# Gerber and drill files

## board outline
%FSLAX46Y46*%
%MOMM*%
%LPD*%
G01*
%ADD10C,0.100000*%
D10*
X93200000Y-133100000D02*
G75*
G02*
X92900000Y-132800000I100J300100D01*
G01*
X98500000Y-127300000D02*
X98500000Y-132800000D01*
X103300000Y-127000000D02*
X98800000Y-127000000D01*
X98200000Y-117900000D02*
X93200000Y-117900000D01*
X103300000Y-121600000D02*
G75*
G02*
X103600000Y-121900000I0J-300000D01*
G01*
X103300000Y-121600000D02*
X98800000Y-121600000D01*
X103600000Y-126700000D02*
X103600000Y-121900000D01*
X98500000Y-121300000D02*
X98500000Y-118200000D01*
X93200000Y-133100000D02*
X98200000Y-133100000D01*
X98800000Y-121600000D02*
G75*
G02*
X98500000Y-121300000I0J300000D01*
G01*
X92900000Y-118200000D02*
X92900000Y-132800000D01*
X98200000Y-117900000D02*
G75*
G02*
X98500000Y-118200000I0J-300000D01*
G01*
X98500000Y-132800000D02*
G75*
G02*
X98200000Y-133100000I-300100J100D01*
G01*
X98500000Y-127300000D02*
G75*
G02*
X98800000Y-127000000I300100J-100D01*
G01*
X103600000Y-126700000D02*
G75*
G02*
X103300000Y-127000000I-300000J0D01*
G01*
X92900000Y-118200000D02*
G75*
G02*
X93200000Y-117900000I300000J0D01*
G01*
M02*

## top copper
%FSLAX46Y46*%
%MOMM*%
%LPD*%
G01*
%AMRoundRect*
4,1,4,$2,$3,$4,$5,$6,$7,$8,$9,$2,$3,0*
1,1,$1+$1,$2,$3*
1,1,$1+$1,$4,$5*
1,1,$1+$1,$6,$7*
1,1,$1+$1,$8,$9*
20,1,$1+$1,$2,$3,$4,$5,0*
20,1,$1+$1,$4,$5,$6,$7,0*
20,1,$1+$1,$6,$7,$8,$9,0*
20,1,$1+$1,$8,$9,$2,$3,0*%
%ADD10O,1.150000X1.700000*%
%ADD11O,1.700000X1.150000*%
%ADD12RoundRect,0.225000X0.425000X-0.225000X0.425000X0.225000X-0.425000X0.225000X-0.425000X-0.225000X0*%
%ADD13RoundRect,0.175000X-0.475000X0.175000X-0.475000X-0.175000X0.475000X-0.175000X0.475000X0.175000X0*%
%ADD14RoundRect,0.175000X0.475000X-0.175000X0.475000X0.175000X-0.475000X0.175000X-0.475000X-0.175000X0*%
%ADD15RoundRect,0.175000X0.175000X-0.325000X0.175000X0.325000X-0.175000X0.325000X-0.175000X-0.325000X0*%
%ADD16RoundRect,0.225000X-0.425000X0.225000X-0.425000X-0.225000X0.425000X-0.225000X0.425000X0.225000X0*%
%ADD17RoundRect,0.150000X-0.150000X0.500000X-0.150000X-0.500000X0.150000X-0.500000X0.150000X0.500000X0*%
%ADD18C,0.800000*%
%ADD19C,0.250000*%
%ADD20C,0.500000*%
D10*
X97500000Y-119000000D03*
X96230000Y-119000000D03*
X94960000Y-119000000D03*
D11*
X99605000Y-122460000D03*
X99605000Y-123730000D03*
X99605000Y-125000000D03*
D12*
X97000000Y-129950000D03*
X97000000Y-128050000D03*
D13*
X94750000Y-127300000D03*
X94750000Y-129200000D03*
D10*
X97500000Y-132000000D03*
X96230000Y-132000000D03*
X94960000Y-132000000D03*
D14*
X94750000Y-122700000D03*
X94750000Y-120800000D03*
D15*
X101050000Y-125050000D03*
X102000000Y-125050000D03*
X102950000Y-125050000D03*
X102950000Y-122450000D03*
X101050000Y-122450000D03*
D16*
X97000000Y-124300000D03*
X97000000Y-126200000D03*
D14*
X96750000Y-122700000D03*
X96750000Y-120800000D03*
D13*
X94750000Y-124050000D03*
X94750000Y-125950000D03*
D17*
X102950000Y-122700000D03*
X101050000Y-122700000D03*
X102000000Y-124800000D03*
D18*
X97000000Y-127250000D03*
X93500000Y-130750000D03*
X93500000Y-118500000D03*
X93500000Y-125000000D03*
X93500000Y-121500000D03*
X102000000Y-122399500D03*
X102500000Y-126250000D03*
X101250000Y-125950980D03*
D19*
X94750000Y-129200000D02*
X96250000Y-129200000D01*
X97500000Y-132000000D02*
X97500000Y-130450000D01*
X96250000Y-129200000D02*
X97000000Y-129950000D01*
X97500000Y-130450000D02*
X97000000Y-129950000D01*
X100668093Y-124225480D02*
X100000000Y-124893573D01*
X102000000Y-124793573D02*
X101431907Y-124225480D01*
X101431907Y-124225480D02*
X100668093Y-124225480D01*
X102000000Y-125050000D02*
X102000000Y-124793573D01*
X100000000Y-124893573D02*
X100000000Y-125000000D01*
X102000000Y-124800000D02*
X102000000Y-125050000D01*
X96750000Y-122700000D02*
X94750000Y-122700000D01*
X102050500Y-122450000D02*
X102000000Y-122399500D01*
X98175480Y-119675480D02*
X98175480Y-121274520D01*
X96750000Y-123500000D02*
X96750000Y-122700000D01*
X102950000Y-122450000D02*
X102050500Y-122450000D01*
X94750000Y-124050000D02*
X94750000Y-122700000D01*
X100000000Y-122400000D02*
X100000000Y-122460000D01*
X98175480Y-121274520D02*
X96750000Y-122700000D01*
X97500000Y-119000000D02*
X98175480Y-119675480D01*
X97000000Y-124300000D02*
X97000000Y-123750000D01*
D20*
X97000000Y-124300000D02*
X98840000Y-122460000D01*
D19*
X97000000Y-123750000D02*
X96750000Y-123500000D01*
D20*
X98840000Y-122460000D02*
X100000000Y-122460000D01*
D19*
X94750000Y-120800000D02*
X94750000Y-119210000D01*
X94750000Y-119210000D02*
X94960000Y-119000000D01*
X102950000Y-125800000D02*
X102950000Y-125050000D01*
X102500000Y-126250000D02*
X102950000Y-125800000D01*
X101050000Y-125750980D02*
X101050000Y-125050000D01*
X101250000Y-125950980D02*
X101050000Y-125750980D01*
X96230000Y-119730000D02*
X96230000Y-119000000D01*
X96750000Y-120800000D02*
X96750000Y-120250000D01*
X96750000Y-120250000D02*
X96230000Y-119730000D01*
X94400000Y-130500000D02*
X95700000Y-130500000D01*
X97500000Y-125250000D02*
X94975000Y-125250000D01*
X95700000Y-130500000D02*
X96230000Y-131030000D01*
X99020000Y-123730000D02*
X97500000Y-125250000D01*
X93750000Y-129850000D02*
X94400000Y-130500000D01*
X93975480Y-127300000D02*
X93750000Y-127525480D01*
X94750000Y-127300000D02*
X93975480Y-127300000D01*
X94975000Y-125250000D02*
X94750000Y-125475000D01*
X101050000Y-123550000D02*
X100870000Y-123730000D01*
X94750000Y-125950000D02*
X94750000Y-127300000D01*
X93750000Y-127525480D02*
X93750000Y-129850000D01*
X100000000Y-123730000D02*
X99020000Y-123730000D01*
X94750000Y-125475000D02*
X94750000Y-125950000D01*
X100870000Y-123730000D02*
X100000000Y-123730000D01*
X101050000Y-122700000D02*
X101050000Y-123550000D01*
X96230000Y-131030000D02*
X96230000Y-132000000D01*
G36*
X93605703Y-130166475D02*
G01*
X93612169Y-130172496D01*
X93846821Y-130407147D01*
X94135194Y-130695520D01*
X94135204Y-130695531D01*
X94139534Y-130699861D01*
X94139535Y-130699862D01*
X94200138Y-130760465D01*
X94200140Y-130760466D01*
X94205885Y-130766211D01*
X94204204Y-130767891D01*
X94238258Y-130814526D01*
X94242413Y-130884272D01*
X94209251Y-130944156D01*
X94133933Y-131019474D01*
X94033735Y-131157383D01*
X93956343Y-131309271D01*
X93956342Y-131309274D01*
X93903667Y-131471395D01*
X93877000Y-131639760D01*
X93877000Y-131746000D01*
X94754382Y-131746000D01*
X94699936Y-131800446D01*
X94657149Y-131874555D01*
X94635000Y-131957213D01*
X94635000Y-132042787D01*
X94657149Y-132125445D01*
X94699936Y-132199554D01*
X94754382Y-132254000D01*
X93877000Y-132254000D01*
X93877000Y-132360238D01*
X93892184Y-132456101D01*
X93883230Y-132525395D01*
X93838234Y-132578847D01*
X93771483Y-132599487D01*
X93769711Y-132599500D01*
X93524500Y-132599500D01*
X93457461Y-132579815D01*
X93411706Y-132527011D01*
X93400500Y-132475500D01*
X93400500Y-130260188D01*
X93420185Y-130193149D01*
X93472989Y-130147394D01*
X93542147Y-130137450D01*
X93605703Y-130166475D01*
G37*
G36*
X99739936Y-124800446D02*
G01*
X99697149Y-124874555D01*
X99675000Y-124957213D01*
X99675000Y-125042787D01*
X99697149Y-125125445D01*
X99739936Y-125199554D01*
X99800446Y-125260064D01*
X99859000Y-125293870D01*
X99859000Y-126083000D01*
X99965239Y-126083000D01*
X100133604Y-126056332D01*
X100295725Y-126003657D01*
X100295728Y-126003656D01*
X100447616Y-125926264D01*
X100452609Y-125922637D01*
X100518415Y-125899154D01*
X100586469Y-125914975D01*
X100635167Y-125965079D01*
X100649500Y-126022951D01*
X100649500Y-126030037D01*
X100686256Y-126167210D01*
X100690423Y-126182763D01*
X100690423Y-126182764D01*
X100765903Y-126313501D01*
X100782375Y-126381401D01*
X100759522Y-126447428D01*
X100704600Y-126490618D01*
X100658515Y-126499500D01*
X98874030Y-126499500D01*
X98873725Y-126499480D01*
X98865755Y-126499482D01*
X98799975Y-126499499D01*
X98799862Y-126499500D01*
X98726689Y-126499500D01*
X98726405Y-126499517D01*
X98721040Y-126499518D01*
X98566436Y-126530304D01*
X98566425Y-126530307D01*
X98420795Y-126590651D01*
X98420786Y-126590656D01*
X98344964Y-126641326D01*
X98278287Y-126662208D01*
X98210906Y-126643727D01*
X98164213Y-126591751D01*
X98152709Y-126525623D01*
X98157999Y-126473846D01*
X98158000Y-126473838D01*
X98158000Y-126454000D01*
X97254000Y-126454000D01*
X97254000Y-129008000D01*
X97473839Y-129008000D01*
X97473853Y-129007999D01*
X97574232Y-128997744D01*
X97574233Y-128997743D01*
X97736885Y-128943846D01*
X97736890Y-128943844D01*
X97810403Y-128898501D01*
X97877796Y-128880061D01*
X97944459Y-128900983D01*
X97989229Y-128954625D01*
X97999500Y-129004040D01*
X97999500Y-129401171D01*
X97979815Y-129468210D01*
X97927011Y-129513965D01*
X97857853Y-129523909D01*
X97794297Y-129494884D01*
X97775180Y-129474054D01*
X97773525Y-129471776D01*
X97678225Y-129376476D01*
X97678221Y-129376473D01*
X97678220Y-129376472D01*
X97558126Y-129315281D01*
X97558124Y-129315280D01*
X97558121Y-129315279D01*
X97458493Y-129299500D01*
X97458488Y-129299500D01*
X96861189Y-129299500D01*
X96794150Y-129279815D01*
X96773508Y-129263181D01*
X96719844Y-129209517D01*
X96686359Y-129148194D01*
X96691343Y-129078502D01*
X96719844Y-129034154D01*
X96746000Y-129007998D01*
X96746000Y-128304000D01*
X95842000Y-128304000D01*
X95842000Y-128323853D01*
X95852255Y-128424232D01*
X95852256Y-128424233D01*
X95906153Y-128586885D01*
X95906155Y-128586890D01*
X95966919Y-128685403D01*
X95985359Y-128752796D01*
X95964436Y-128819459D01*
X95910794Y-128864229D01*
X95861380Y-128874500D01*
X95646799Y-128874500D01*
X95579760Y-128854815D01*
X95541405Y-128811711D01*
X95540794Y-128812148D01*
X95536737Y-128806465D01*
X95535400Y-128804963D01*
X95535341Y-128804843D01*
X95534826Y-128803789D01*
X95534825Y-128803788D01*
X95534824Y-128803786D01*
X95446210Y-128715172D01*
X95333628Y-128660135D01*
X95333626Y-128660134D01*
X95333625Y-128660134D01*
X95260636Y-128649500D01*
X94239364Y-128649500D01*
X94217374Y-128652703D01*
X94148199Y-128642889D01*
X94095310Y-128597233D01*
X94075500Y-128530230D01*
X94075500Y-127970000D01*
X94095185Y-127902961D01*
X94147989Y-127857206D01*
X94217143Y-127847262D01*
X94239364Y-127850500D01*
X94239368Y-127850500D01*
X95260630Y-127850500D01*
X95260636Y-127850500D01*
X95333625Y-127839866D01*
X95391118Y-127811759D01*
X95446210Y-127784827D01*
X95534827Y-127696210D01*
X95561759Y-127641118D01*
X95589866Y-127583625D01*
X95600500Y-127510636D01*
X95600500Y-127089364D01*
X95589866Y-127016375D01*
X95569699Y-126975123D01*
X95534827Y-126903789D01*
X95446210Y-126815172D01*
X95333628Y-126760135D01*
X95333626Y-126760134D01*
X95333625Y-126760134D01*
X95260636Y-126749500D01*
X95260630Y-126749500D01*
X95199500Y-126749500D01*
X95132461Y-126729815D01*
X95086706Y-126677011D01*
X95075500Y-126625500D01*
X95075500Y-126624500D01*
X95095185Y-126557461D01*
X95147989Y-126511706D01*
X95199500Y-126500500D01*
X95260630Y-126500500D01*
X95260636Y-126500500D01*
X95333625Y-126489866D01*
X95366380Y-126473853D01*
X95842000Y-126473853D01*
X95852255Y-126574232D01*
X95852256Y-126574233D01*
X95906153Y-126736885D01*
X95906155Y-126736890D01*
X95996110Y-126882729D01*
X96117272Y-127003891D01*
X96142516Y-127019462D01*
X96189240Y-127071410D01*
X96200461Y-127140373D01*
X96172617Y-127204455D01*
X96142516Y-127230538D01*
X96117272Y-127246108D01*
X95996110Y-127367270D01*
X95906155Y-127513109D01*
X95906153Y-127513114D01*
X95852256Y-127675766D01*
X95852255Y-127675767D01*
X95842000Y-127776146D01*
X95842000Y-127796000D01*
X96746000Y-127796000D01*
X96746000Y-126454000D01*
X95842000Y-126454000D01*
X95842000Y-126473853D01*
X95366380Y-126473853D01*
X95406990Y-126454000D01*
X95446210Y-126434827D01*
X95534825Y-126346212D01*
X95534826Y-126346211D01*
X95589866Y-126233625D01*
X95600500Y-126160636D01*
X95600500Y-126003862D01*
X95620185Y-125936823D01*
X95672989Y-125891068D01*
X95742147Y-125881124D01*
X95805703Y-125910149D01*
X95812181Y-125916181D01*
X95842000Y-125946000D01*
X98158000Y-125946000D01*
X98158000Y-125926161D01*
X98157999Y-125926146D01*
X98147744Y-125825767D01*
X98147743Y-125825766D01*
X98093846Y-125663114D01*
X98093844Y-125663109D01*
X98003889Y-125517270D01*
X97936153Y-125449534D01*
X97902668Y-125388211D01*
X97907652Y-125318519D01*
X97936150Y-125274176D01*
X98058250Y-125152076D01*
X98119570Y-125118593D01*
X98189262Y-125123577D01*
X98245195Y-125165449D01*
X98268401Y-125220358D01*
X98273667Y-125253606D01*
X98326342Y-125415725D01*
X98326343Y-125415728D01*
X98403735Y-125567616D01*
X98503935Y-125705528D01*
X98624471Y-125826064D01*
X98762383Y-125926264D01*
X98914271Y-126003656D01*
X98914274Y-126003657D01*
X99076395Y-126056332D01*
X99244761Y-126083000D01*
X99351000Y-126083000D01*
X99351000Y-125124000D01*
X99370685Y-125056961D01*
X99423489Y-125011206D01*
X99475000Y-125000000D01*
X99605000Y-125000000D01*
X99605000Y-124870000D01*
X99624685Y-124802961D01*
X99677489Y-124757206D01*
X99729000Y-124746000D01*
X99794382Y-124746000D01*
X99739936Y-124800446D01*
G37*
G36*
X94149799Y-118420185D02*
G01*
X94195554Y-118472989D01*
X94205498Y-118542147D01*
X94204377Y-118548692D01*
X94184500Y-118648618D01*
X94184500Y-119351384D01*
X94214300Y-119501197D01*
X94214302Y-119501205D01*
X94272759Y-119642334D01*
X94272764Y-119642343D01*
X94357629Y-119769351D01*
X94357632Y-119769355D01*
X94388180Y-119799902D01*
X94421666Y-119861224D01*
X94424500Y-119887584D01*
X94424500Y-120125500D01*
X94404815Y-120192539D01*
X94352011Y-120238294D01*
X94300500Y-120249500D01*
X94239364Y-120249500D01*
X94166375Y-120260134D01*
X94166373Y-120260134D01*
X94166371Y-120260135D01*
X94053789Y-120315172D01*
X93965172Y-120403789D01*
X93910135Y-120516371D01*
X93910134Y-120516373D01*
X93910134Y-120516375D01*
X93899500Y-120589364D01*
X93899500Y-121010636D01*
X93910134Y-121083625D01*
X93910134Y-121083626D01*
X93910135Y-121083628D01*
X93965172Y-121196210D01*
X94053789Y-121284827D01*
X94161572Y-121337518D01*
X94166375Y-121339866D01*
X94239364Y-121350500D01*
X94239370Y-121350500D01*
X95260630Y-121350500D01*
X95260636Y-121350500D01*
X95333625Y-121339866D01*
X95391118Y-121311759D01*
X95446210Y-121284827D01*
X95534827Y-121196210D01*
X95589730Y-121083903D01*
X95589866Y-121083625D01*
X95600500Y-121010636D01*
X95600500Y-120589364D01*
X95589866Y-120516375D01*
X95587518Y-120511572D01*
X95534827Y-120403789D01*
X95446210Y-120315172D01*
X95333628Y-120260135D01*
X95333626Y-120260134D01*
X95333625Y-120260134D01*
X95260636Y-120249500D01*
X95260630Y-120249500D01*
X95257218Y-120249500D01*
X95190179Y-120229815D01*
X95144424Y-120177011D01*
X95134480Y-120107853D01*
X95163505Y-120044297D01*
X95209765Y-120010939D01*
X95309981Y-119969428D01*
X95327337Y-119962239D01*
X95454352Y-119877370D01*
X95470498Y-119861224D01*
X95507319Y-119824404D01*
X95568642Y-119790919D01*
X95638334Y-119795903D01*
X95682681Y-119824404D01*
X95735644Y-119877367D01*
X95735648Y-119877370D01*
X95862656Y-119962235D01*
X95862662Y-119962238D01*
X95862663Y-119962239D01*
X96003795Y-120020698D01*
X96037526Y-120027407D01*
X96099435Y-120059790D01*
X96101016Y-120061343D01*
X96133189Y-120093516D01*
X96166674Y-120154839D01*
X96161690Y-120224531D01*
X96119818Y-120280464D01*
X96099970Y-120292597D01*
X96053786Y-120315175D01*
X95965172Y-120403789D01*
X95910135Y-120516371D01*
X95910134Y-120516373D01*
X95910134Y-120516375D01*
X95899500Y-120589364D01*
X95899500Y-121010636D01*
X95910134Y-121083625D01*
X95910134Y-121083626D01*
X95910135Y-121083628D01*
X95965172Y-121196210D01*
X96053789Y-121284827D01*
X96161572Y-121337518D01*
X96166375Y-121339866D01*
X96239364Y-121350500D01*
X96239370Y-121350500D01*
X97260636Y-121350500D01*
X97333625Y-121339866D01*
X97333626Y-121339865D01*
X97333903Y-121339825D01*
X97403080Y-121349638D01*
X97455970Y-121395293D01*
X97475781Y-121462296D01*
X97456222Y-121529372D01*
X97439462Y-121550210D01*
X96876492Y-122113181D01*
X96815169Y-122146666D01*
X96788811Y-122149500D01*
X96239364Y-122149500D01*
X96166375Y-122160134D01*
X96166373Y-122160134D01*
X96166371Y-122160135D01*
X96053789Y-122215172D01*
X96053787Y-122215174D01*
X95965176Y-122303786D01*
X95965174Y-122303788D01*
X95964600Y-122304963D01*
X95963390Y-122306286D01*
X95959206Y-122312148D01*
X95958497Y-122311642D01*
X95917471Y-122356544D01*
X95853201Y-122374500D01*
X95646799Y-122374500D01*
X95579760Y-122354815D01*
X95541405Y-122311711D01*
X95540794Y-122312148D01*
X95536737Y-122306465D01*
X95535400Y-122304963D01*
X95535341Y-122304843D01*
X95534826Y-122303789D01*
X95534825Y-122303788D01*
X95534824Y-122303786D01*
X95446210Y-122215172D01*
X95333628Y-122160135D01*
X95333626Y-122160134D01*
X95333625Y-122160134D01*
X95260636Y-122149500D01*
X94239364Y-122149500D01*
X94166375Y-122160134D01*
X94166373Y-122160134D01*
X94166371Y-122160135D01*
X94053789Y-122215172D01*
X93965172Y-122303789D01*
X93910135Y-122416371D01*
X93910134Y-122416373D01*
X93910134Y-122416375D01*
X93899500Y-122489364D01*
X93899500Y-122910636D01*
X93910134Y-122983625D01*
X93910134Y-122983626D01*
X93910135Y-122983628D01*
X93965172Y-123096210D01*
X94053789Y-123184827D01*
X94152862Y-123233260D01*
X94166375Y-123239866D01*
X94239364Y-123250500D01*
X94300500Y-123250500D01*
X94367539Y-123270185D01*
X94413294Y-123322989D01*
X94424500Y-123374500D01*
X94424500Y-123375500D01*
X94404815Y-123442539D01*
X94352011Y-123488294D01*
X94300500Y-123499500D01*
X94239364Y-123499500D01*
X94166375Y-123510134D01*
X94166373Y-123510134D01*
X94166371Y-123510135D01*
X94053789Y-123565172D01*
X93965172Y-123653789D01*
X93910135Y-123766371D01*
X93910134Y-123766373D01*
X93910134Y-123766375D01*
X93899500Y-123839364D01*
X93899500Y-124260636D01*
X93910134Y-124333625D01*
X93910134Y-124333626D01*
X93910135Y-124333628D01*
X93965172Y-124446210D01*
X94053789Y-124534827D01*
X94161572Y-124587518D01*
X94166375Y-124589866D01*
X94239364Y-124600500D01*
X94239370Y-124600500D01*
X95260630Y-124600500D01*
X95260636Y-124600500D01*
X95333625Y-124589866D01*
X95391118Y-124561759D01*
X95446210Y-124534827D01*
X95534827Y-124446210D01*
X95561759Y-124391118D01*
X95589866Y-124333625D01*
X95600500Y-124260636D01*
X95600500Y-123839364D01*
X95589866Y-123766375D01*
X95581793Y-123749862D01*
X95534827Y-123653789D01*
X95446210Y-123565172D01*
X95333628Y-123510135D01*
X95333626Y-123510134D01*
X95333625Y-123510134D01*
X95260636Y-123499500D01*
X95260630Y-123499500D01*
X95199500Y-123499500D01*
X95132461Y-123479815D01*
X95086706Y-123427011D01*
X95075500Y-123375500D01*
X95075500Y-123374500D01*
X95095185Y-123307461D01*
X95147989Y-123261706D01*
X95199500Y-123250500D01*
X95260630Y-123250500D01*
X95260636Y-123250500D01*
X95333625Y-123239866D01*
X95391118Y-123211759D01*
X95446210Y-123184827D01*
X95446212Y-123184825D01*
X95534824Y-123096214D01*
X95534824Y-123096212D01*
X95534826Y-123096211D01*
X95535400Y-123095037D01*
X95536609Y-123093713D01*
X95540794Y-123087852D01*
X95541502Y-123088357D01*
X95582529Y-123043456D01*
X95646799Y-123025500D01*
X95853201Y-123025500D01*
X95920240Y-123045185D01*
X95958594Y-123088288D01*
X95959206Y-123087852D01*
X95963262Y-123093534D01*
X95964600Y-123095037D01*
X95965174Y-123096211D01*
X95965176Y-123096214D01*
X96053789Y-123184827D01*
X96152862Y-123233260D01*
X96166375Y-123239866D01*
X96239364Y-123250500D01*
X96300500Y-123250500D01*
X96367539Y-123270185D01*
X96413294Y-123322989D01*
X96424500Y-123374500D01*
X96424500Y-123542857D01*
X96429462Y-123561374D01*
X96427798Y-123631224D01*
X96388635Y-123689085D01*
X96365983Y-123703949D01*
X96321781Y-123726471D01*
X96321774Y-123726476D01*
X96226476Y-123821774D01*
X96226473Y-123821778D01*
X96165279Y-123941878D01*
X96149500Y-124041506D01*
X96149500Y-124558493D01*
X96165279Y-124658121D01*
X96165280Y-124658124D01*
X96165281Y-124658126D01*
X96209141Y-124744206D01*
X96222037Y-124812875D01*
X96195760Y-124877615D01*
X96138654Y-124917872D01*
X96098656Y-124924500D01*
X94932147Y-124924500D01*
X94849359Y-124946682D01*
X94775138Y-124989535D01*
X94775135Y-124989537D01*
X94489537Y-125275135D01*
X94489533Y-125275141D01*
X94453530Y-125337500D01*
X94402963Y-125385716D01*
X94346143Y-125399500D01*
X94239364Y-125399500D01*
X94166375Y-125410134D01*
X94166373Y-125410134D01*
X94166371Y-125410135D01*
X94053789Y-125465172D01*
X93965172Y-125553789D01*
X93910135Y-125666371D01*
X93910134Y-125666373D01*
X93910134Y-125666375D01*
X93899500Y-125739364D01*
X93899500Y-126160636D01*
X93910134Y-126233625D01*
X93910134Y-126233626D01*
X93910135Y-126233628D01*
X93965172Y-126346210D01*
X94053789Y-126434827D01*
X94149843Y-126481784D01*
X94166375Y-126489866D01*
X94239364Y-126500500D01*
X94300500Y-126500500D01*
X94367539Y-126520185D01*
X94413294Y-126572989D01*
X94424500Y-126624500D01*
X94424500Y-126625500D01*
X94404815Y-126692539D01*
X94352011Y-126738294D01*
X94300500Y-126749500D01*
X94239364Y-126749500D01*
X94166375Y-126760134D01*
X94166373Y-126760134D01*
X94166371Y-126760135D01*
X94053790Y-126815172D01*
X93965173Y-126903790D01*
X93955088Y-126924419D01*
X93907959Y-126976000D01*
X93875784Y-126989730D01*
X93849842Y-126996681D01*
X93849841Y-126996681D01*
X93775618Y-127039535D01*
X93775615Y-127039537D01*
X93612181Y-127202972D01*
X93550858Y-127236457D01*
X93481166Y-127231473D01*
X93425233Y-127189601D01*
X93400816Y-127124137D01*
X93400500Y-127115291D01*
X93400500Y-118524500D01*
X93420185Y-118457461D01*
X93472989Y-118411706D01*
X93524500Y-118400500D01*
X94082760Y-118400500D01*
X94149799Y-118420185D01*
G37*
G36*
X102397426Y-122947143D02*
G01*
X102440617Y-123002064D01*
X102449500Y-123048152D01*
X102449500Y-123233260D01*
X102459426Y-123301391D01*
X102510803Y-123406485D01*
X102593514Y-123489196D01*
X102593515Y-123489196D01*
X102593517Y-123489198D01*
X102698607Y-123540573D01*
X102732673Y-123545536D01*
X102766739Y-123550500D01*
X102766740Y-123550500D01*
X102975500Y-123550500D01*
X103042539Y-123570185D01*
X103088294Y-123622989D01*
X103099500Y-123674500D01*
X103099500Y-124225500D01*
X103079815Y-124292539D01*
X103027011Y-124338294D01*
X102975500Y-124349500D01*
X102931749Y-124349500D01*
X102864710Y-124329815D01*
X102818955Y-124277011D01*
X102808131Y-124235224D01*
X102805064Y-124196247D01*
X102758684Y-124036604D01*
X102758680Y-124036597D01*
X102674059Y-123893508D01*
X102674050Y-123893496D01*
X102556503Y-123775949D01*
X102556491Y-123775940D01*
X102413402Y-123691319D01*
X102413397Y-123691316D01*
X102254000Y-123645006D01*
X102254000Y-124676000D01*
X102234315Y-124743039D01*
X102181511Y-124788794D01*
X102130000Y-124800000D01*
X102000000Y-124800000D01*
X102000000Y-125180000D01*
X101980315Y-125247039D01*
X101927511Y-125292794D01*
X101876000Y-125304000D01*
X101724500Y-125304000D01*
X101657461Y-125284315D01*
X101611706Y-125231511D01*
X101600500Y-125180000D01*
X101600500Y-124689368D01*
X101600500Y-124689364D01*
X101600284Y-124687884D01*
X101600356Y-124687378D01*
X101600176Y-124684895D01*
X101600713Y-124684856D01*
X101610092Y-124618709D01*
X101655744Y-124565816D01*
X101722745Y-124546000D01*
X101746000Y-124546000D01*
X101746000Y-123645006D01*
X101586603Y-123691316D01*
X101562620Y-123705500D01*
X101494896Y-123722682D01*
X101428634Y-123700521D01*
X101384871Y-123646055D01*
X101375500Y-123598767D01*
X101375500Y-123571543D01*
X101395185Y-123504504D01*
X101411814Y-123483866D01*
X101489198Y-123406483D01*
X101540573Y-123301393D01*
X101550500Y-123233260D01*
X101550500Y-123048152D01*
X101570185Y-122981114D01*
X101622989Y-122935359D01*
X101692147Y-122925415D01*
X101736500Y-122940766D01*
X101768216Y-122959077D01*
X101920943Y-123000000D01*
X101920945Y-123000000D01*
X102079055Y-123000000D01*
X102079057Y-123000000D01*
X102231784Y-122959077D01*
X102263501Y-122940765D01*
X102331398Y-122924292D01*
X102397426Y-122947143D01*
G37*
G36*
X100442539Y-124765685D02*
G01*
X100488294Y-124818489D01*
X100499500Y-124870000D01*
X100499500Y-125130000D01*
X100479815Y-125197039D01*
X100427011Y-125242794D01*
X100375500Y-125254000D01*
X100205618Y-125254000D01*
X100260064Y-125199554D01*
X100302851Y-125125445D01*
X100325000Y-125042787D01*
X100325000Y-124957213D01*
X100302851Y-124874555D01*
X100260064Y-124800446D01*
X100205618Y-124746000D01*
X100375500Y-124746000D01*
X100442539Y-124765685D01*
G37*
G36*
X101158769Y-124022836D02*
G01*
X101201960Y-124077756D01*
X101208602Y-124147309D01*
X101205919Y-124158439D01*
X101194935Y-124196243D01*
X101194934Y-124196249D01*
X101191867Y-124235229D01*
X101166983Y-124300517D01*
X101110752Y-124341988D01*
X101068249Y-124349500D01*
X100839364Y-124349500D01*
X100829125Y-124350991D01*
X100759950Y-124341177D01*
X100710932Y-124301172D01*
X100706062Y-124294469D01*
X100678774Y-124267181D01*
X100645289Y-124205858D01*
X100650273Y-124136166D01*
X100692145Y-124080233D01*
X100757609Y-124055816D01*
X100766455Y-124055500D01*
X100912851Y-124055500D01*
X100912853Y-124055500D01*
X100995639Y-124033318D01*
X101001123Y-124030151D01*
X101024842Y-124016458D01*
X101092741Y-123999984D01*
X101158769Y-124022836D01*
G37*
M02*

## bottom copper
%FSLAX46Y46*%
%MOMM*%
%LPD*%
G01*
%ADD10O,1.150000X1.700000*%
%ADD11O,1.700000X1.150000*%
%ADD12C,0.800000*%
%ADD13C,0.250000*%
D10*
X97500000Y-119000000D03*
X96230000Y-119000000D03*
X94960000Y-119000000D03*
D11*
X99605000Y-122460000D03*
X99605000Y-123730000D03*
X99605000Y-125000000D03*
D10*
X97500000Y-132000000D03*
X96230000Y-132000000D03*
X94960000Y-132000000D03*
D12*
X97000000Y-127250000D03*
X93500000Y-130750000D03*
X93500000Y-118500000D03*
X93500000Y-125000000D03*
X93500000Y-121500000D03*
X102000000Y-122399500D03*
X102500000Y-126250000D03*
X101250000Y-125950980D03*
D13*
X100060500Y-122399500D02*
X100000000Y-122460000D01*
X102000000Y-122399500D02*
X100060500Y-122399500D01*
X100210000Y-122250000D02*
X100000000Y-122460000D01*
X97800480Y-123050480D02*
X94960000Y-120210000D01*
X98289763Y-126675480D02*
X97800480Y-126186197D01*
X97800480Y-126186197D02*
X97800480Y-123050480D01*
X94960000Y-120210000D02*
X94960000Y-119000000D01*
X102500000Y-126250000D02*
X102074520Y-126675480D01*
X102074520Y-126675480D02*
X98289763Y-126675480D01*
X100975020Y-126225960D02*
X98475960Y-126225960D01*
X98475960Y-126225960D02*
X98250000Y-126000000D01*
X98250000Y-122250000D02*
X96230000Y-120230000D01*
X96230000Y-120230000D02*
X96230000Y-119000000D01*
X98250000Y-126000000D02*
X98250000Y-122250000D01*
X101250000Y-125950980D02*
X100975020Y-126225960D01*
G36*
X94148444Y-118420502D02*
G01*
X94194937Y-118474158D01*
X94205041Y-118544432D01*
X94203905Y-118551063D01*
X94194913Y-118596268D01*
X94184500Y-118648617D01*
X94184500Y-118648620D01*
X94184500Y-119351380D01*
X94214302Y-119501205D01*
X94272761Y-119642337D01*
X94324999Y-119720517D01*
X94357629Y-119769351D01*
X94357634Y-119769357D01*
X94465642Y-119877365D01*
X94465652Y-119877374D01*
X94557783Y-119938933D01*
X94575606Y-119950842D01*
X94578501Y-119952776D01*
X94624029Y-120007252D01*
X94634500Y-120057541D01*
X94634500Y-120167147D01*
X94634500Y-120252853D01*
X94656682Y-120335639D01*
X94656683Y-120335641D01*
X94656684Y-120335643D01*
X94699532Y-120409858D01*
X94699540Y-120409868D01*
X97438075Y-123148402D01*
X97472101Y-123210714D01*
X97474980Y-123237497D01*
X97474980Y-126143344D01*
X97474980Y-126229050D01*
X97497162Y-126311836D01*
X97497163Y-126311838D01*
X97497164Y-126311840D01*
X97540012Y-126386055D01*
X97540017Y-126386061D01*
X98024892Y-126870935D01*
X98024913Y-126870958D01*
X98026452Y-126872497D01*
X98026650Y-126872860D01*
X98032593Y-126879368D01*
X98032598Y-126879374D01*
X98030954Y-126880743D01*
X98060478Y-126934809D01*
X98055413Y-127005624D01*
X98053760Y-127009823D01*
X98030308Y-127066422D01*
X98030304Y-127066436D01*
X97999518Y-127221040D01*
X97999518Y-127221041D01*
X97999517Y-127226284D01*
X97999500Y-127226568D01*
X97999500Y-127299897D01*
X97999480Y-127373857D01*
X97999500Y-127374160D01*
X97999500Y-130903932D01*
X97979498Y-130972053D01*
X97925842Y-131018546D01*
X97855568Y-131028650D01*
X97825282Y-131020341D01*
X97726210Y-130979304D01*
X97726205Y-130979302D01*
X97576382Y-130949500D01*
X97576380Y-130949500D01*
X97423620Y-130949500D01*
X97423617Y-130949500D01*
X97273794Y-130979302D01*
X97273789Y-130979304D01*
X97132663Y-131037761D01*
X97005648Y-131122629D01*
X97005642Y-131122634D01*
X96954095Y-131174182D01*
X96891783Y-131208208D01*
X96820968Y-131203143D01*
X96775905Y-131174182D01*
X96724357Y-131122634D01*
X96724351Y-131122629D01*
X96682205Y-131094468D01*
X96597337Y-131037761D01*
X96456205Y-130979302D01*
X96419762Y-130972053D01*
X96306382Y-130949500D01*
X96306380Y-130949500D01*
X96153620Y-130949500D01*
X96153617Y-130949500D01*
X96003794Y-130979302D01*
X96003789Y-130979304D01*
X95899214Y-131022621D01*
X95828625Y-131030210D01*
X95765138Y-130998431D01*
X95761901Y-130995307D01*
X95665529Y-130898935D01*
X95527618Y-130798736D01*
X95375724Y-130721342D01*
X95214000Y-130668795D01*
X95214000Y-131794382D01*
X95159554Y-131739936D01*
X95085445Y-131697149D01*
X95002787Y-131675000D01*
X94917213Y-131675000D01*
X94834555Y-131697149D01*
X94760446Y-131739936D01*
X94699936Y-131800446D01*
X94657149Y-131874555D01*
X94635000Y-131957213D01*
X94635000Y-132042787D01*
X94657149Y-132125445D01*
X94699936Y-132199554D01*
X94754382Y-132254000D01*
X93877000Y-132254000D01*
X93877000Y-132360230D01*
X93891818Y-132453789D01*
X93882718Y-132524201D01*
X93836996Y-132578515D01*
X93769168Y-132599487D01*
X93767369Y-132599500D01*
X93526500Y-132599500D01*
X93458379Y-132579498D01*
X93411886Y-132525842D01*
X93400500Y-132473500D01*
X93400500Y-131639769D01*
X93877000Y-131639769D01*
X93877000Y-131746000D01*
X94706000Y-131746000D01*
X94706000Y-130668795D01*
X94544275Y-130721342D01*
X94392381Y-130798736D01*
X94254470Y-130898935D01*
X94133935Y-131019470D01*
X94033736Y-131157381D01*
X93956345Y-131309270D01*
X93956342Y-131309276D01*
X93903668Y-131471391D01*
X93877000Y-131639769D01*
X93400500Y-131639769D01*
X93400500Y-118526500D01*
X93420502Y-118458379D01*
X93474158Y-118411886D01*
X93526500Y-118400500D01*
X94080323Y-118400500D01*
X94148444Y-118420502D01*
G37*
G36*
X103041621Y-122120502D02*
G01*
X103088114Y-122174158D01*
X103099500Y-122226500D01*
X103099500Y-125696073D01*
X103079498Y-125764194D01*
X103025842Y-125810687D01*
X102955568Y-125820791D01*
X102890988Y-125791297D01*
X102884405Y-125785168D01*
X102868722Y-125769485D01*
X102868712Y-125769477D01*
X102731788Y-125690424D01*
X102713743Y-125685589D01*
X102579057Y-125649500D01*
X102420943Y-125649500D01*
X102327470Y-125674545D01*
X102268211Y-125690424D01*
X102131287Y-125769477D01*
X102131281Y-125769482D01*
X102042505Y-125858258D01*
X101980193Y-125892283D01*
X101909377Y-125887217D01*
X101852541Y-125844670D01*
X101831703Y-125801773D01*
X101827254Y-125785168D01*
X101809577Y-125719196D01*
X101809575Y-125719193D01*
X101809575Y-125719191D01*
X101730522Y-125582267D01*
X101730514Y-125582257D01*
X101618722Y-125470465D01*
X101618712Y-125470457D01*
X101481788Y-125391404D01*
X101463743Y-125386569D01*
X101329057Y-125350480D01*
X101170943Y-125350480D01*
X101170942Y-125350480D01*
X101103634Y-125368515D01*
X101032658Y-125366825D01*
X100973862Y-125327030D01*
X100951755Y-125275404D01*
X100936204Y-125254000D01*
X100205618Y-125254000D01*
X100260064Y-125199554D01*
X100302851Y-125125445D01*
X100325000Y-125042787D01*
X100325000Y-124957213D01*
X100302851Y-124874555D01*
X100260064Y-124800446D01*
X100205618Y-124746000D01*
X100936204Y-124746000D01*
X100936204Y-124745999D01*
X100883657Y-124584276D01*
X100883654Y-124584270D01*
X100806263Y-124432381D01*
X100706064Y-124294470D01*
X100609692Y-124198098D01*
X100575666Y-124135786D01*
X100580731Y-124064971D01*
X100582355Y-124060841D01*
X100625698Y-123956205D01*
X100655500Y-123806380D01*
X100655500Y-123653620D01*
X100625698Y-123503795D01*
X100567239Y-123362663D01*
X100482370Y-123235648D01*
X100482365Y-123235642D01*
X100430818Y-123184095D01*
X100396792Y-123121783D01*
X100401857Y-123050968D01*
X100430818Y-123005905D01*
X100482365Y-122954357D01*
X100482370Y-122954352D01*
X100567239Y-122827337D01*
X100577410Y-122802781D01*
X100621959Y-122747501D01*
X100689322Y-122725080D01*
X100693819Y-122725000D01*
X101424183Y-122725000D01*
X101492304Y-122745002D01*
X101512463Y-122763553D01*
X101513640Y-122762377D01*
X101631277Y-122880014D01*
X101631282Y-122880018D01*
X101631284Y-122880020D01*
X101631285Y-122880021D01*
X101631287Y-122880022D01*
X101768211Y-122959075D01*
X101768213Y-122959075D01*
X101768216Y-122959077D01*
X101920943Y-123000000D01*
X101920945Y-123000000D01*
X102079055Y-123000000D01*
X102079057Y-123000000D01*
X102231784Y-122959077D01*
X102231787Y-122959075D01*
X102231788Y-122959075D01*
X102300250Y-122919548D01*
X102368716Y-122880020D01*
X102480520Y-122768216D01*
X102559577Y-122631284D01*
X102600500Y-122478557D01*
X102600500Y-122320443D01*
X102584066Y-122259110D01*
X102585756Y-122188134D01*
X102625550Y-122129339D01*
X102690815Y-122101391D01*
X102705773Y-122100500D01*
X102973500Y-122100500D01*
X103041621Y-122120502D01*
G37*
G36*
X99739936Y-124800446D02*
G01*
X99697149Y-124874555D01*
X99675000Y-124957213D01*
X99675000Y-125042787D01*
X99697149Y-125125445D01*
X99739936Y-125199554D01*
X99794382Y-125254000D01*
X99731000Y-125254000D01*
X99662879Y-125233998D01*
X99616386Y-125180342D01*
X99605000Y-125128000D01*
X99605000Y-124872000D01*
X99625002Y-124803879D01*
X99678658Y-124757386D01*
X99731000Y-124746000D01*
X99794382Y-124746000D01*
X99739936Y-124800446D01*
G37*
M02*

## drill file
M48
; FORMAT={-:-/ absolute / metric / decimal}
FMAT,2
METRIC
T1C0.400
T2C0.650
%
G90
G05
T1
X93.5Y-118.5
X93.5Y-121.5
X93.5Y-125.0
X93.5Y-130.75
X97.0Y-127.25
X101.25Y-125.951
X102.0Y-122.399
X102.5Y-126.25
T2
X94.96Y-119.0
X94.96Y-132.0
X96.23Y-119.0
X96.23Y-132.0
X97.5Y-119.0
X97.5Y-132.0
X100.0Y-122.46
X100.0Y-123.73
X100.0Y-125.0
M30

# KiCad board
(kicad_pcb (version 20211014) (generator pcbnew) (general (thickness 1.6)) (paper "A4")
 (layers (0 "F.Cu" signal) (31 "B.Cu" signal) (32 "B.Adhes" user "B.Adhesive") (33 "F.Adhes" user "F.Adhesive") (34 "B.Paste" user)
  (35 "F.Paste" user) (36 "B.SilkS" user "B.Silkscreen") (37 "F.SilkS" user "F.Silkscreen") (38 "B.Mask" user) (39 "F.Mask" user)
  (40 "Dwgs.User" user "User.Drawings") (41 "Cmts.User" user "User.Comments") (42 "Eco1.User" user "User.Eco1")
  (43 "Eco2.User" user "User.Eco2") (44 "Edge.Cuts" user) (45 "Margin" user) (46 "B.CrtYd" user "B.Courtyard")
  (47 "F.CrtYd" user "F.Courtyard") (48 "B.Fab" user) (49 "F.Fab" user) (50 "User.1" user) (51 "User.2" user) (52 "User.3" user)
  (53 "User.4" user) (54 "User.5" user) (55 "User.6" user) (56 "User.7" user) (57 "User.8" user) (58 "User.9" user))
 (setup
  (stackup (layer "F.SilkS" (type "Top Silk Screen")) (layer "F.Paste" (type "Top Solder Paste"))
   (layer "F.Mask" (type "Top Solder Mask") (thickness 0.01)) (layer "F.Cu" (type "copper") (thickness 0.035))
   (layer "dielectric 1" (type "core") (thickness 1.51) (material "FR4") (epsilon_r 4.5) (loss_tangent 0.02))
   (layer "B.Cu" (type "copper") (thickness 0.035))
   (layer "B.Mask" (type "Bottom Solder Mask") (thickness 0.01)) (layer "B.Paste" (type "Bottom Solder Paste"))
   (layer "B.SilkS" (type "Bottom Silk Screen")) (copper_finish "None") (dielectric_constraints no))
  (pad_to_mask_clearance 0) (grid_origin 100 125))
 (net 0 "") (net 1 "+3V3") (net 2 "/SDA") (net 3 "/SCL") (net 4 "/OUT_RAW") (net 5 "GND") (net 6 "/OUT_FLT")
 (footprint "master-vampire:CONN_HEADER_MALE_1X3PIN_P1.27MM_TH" (layer "F.Cu") (at 97.5 119 180)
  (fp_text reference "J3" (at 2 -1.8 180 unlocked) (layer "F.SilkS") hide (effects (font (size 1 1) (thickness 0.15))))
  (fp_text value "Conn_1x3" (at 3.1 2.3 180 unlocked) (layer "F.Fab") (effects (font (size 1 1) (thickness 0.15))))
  (pad "1" thru_hole oval (at 0 0 180) (size 1.15 1.7) (drill 0.65) (layers *.Cu *.Mask) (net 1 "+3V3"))
  (pad "2" thru_hole oval (at 1.27 0 180) (size 1.15 1.7) (drill 0.65) (layers *.Cu *.Mask) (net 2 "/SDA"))
  (pad "3" thru_hole oval (at 2.54 0 180) (size 1.15 1.7) (drill 0.65) (layers *.Cu *.Mask) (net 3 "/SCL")))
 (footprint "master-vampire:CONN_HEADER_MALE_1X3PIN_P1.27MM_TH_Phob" (layer "F.Cu") (at 100 122.46 -90)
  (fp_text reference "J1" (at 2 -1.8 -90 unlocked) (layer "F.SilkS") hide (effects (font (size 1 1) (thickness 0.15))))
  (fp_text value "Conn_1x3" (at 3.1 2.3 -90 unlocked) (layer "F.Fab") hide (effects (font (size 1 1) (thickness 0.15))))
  (pad "1" thru_hole oval (at 0 0 270) (size 1.15 1.7) (drill 0.65 (offset 0 0.395)) (layers *.Cu *.Mask) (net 1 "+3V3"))
  (pad "2" thru_hole oval (at 1.27 0 270) (size 1.15 1.7) (drill 0.65 (offset 0 0.395)) (layers *.Cu *.Mask) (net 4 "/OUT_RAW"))
  (pad "3" thru_hole oval (at 2.54 0 270) (size 1.15 1.7) (drill 0.65 (offset 0 0.395)) (layers *.Cu *.Mask) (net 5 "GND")))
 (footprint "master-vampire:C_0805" (layer "F.Cu") (at 97 129 90)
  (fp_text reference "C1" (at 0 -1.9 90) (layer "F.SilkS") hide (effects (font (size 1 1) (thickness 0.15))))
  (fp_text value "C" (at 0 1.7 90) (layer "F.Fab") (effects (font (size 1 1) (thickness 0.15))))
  (pad "1" smd roundrect (at -0.95 0 90) (size 0.9 1.3) (layers "F.Cu" "F.Paste" "F.Mask") (roundrect_rratio 0.25) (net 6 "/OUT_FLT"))
  (pad "2" smd roundrect (at 0.95 0 90) (size 0.9 1.3) (layers "F.Cu" "F.Paste" "F.Mask") (roundrect_rratio 0.25) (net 5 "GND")))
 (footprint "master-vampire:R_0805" (layer "F.Cu") (at 94.75 128.25 -90)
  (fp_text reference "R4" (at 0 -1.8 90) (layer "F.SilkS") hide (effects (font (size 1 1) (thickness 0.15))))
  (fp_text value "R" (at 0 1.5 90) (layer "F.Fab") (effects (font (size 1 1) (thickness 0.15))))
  (pad "1" smd roundrect (at -0.95 0 270) (size 0.7 1.3) (layers "F.Cu" "F.Paste" "F.Mask") (roundrect_rratio 0.25) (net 4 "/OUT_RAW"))
  (pad "2" smd roundrect (at 0.95 0 270) (size 0.7 1.3) (layers "F.Cu" "F.Paste" "F.Mask") (roundrect_rratio 0.25) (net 6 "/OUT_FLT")))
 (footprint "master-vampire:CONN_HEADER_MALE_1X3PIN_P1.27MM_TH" (layer "F.Cu") (at 97.5 132 180)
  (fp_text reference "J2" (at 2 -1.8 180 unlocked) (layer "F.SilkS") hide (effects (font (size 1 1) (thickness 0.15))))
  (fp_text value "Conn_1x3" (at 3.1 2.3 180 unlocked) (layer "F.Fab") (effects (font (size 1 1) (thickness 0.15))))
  (pad "1" thru_hole oval (at 0 0 180) (size 1.15 1.7) (drill 0.65) (layers *.Cu *.Mask) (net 6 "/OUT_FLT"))
  (pad "2" thru_hole oval (at 1.27 0 180) (size 1.15 1.7) (drill 0.65) (layers *.Cu *.Mask) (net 4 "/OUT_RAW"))
  (pad "3" thru_hole oval (at 2.54 0 180) (size 1.15 1.7) (drill 0.65) (layers *.Cu *.Mask) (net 5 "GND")))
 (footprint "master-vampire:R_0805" (layer "F.Cu") (at 94.75 121.75 90)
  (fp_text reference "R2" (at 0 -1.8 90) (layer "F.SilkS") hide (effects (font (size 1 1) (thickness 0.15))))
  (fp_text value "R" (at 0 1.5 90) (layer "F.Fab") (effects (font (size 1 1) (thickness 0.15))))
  (pad "1" smd roundrect (at -0.95 0 90) (size 0.7 1.3) (layers "F.Cu" "F.Paste" "F.Mask") (roundrect_rratio 0.25) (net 1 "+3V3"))
  (pad "2" smd roundrect (at 0.95 0 90) (size 0.7 1.3) (layers "F.Cu" "F.Paste" "F.Mask") (roundrect_rratio 0.25) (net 3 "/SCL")))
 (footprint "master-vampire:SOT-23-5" (layer "F.Cu") (at 102 123.75 90)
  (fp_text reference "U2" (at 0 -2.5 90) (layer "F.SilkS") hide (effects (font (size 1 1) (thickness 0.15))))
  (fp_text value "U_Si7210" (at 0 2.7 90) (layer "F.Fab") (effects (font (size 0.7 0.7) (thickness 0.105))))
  (pad "1" smd roundrect (at -1.3 -0.95 90) (size 1 0.7) (layers "F.Cu" "F.Paste" "F.Mask") (roundrect_rratio 0.25) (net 2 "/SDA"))
  (pad "2" smd roundrect (at -1.3 0 90) (size 1 0.7) (layers "F.Cu" "F.Paste" "F.Mask") (roundrect_rratio 0.25) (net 5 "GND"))
  (pad "3" smd roundrect (at -1.3 0.95 90) (size 1 0.7) (layers "F.Cu" "F.Paste" "F.Mask") (roundrect_rratio 0.25) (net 3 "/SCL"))
  (pad "4" smd roundrect (at 1.3 0.95 90) (size 1 0.7) (layers "F.Cu" "F.Paste" "F.Mask") (roundrect_rratio 0.25) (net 1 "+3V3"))
  (pad "5" smd roundrect (at 1.3 -0.95 90) (size 1 0.7) (layers "F.Cu" "F.Paste" "F.Mask") (roundrect_rratio 0.25) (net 4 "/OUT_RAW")))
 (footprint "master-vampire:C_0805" (layer "F.Cu") (at 97 125.25 -90)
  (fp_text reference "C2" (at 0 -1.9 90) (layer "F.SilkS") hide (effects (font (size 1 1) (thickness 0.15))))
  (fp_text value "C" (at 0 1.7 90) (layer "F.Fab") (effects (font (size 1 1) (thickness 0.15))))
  (pad "1" smd roundrect (at -0.95 0 270) (size 0.9 1.3) (layers "F.Cu" "F.Paste" "F.Mask") (roundrect_rratio 0.25) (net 1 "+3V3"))
  (pad "2" smd roundrect (at 0.95 0 270) (size 0.9 1.3) (layers "F.Cu" "F.Paste" "F.Mask") (roundrect_rratio 0.25) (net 5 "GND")))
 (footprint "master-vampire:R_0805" (layer "F.Cu") (at 96.75 121.75 90)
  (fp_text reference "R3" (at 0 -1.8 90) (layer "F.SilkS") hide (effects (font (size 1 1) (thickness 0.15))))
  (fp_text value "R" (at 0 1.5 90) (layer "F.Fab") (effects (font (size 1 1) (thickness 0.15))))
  (pad "1" smd roundrect (at -0.95 0 90) (size 0.7 1.3) (layers "F.Cu" "F.Paste" "F.Mask") (roundrect_rratio 0.25) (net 1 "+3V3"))
  (pad "2" smd roundrect (at 0.95 0 90) (size 0.7 1.3) (layers "F.Cu" "F.Paste" "F.Mask") (roundrect_rratio 0.25) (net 2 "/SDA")))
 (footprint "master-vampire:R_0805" (layer "F.Cu") (at 94.75 125 -90)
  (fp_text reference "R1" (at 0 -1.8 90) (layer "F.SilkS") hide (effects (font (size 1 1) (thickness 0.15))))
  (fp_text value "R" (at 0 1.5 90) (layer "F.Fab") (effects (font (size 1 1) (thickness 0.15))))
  (pad "1" smd roundrect (at -0.95 0 270) (size 0.7 1.3) (layers "F.Cu" "F.Paste" "F.Mask") (roundrect_rratio 0.25) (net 1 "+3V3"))
  (pad "2" smd roundrect (at 0.95 0 270) (size 0.7 1.3) (layers "F.Cu" "F.Paste" "F.Mask") (roundrect_rratio 0.25) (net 4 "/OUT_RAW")))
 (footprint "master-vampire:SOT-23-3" (layer "F.Cu") (at 102 123.75 -90)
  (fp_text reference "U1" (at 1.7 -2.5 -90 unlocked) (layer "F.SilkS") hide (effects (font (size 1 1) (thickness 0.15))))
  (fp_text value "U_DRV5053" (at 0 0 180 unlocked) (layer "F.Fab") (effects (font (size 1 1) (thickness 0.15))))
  (pad "1" smd roundrect (at -1.05 -0.95 270) (size 1.3 0.6) (layers "F.Cu" "F.Paste" "F.Mask") (roundrect_rratio 0.25) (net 1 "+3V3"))
  (pad "2" smd roundrect (at -1.05 0.95 270) (size 1.3 0.6) (layers "F.Cu" "F.Paste" "F.Mask") (roundrect_rratio 0.25) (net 4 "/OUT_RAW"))
  (pad "3" smd roundrect (at 1.05 0 270) (size 1.3 0.6) (layers "F.Cu" "F.Paste" "F.Mask") (roundrect_rratio 0.25) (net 5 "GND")))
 (gr_arc (start 93.2 133.1) (mid 92.987897 133.012103) (end 92.9 132.8) (layer "Edge.Cuts") (width 0.1))
 (gr_line (start 98.5 127.3) (end 98.5 132.8) (layer "Edge.Cuts") (width 0.1))
 (gr_line (start 103.3 127) (end 98.8 127) (layer "Edge.Cuts") (width 0.1))
 (gr_line (start 98.2 117.9) (end 93.2 117.9) (layer "Edge.Cuts") (width 0.1))
 (gr_arc (start 103.3 121.6) (mid 103.512132 121.687868) (end 103.6 121.9) (layer "Edge.Cuts") (width 0.1))
 (gr_line (start 103.3 121.6) (end 98.8 121.6) (layer "Edge.Cuts") (width 0.1))
 (gr_line (start 103.6 126.7) (end 103.6 121.9) (layer "Edge.Cuts") (width 0.1))
 (gr_line (start 98.5 121.3) (end 98.5 118.2) (layer "Edge.Cuts") (width 0.1))
 (gr_line (start 93.2 133.1) (end 98.2 133.1) (layer "Edge.Cuts") (width 0.1))
 (gr_arc (start 98.8 121.6) (mid 98.587868 121.512132) (end 98.5 121.3) (layer "Edge.Cuts") (width 0.1))
 (gr_line (start 92.9 118.2) (end 92.9 132.8) (layer "Edge.Cuts") (width 0.1))
 (gr_arc (start 98.2 117.9) (mid 98.412132 117.987868) (end 98.5 118.2) (layer "Edge.Cuts") (width 0.1))
 (gr_arc (start 98.5 132.8) (mid 98.412103 133.012103) (end 98.2 133.1) (layer "Edge.Cuts") (width 0.1))
 (gr_arc (start 98.5 127.3) (mid 98.587884 127.0879) (end 98.8 127) (layer "Edge.Cuts") (width 0.1))
 (gr_arc (start 103.6 126.7) (mid 103.512132 126.912132) (end 103.3 127) (layer "Edge.Cuts") (width 0.1))
 (gr_arc (start 92.9 118.2) (mid 92.987868 117.987868) (end 93.2 117.9) (layer "Edge.Cuts") (width 0.1))
 (segment (start 94.75 129.2) (end 96.25 129.2) (width 0.25) (layer "F.Cu") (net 6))
 (segment (start 97.5 132) (end 97.5 130.45) (width 0.25) (layer "F.Cu") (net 6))
 (segment (start 96.25 129.2) (end 97 129.95) (width 0.25) (layer "F.Cu") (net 6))
 (segment (start 97.5 130.45) (end 97 129.95) (width 0.25) (layer "F.Cu") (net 6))
 (segment (start 100.668093 124.22548) (end 100 124.893573) (width 0.25) (layer "F.Cu") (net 5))
 (segment (start 102 124.793573) (end 101.431907 124.22548) (width 0.25) (layer "F.Cu") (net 5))
 (segment (start 101.431907 124.22548) (end 100.668093 124.22548) (width 0.25) (layer "F.Cu") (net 5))
 (segment (start 102 125.05) (end 102 124.793573) (width 0.25) (layer "F.Cu") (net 5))
 (segment (start 100 124.893573) (end 100 125) (width 0.25) (layer "F.Cu") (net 5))
 (segment (start 102 124.8) (end 102 125.05) (width 0.25) (layer "F.Cu") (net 5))
 (via (at 97 127.25) (size 0.8) (drill 0.4) (layers "F.Cu" "B.Cu") (free) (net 5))
 (via (at 93.5 130.75) (size 0.8) (drill 0.4) (layers "F.Cu" "B.Cu") (free) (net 5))
 (via (at 93.5 118.5) (size 0.8) (drill 0.4) (layers "F.Cu" "B.Cu") (free) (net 5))
 (via (at 93.5 125) (size 0.8) (drill 0.4) (layers "F.Cu" "B.Cu") (free) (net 5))
 (via (at 93.5 121.5) (size 0.8) (drill 0.4) (layers "F.Cu" "B.Cu") (free) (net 5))
 (segment (start 96.75 122.7) (end 94.75 122.7) (width 0.25) (layer "F.Cu") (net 1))
 (segment (start 102.0505 122.45) (end 102 122.3995) (width 0.25) (layer "F.Cu") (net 1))
 (segment (start 98.17548 119.67548) (end 98.17548 121.27452) (width 0.25) (layer "F.Cu") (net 1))
 (segment (start 96.75 123.5) (end 96.75 122.7) (width 0.25) (layer "F.Cu") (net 1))
 (segment (start 102.95 122.45) (end 102.0505 122.45) (width 0.25) (layer "F.Cu") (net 1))
 (segment (start 94.75 124.05) (end 94.75 122.7) (width 0.25) (layer "F.Cu") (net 1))
 (segment (start 100 122.4) (end 100 122.46) (width 0.25) (layer "F.Cu") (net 1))
 (segment (start 98.17548 121.27452) (end 96.75 122.7) (width 0.25) (layer "F.Cu") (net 1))
 (segment (start 97.5 119) (end 98.17548 119.67548) (width 0.25) (layer "F.Cu") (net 1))
 (segment (start 97 124.3) (end 97 123.75) (width 0.25) (layer "F.Cu") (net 1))
 (segment (start 97 124.3) (end 98.84 122.46) (width 0.5) (layer "F.Cu") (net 1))
 (segment (start 97 123.75) (end 96.75 123.5) (width 0.25) (layer "F.Cu") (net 1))
 (segment (start 98.84 122.46) (end 100 122.46) (width 0.5) (layer "F.Cu") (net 1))
 (via (at 102 122.3995) (size 0.8) (drill 0.4) (layers "F.Cu" "B.Cu") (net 1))
 (segment (start 100.0605 122.3995) (end 100 122.46) (width 0.25) (layer "B.Cu") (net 1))
 (segment (start 102 122.3995) (end 100.0605 122.3995) (width 0.25) (layer "B.Cu") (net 1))
 (segment (start 100.21 122.25) (end 100 122.46) (width 0.25) (layer "B.Cu") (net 1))
 (segment (start 94.75 120.8) (end 94.75 119.21) (width 0.25) (layer "F.Cu") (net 3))
 (segment (start 94.75 119.21) (end 94.96 119) (width 0.25) (layer "F.Cu") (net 3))
 (segment (start 102.95 125.8) (end 102.95 125.05) (width 0.25) (layer "F.Cu") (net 3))
 (segment (start 102.5 126.25) (end 102.95 125.8) (width 0.25) (layer "F.Cu") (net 3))
 (via (at 102.5 126.25) (size 0.8) (drill 0.4) (layers "F.Cu" "B.Cu") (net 3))
 (segment (start 97.80048 123.05048) (end 94.96 120.21) (width 0.25) (layer "B.Cu") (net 3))
 (segment (start 98.289763 126.67548) (end 97.80048 126.186197) (width 0.25) (layer "B.Cu") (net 3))
 (segment (start 97.80048 126.186197) (end 97.80048 123.05048) (width 0.25) (layer "B.Cu") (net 3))
 (segment (start 94.96 120.21) (end 94.96 119) (width 0.25) (layer "B.Cu") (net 3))
 (segment (start 102.5 126.25) (end 102.07452 126.67548) (width 0.25) (layer "B.Cu") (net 3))
 (segment (start 102.07452 126.67548) (end 98.289763 126.67548) (width 0.25) (layer "B.Cu") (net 3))
 (segment (start 101.05 125.75098) (end 101.05 125.05) (width 0.25) (layer "F.Cu") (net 2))
 (segment (start 101.25 125.95098) (end 101.05 125.75098) (width 0.25) (layer "F.Cu") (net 2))
 (segment (start 96.23 119.73) (end 96.23 119) (width 0.25) (layer "F.Cu") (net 2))
 (segment (start 96.75 120.8) (end 96.75 120.25) (width 0.25) (layer "F.Cu") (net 2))
 (segment (start 96.75 120.25) (end 96.23 119.73) (width 0.25) (layer "F.Cu") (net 2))
 (via (at 101.25 125.95098) (size 0.8) (drill 0.4) (layers "F.Cu" "B.Cu") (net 2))
 (segment (start 100.97502 126.22596) (end 98.47596 126.22596) (width 0.25) (layer "B.Cu") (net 2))
 (segment (start 98.47596 126.22596) (end 98.25 126) (width 0.25) (layer "B.Cu") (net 2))
 (segment (start 98.25 122.25) (end 96.23 120.23) (width 0.25) (layer "B.Cu") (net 2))
 (segment (start 96.23 120.23) (end 96.23 119) (width 0.25) (layer "B.Cu") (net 2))
 (segment (start 98.25 126) (end 98.25 122.25) (width 0.25) (layer "B.Cu") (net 2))
 (segment (start 101.25 125.95098) (end 100.97502 126.22596) (width 0.25) (layer "B.Cu") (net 2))
 (segment (start 94.4 130.5) (end 95.7 130.5) (width 0.25) (layer "F.Cu") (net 4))
 (segment (start 97.5 125.25) (end 94.975 125.25) (width 0.25) (layer "F.Cu") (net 4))
 (segment (start 95.7 130.5) (end 96.23 131.03) (width 0.25) (layer "F.Cu") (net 4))
 (segment (start 99.02 123.73) (end 97.5 125.25) (width 0.25) (layer "F.Cu") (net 4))
 (segment (start 93.75 129.85) (end 94.4 130.5) (width 0.25) (layer "F.Cu") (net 4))
 (segment (start 93.97548 127.3) (end 93.75 127.52548) (width 0.25) (layer "F.Cu") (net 4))
 (segment (start 94.75 127.3) (end 93.97548 127.3) (width 0.25) (layer "F.Cu") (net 4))
 (segment (start 94.975 125.25) (end 94.75 125.475) (width 0.25) (layer "F.Cu") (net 4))
 (segment (start 101.05 123.55) (end 100.87 123.73) (width 0.25) (layer "F.Cu") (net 4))
 (segment (start 94.75 125.95) (end 94.75 127.3) (width 0.25) (layer "F.Cu") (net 4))
 (segment (start 93.75 127.52548) (end 93.75 129.85) (width 0.25) (layer "F.Cu") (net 4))
 (segment (start 100 123.73) (end 99.02 123.73) (width 0.25) (layer "F.Cu") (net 4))
 (segment (start 94.75 125.475) (end 94.75 125.95) (width 0.25) (layer "F.Cu") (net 4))
 (segment (start 100.87 123.73) (end 100 123.73) (width 0.25) (layer "F.Cu") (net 4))
 (segment (start 101.05 122.7) (end 101.05 123.55) (width 0.25) (layer "F.Cu") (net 4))
 (segment (start 96.23 131.03) (end 96.23 132) (width 0.25) (layer "F.Cu") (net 4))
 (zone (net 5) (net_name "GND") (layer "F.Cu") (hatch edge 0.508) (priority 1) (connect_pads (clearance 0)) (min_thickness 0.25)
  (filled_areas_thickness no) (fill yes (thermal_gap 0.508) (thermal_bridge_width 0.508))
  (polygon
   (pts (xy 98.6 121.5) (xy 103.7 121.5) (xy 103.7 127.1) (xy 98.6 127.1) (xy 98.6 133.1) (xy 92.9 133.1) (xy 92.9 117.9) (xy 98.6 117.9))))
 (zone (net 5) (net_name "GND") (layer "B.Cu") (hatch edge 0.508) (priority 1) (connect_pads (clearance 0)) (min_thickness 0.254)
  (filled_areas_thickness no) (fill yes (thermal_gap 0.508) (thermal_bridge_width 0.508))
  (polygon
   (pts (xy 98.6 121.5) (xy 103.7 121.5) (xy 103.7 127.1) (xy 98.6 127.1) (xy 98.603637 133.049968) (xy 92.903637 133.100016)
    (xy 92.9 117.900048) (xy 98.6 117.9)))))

